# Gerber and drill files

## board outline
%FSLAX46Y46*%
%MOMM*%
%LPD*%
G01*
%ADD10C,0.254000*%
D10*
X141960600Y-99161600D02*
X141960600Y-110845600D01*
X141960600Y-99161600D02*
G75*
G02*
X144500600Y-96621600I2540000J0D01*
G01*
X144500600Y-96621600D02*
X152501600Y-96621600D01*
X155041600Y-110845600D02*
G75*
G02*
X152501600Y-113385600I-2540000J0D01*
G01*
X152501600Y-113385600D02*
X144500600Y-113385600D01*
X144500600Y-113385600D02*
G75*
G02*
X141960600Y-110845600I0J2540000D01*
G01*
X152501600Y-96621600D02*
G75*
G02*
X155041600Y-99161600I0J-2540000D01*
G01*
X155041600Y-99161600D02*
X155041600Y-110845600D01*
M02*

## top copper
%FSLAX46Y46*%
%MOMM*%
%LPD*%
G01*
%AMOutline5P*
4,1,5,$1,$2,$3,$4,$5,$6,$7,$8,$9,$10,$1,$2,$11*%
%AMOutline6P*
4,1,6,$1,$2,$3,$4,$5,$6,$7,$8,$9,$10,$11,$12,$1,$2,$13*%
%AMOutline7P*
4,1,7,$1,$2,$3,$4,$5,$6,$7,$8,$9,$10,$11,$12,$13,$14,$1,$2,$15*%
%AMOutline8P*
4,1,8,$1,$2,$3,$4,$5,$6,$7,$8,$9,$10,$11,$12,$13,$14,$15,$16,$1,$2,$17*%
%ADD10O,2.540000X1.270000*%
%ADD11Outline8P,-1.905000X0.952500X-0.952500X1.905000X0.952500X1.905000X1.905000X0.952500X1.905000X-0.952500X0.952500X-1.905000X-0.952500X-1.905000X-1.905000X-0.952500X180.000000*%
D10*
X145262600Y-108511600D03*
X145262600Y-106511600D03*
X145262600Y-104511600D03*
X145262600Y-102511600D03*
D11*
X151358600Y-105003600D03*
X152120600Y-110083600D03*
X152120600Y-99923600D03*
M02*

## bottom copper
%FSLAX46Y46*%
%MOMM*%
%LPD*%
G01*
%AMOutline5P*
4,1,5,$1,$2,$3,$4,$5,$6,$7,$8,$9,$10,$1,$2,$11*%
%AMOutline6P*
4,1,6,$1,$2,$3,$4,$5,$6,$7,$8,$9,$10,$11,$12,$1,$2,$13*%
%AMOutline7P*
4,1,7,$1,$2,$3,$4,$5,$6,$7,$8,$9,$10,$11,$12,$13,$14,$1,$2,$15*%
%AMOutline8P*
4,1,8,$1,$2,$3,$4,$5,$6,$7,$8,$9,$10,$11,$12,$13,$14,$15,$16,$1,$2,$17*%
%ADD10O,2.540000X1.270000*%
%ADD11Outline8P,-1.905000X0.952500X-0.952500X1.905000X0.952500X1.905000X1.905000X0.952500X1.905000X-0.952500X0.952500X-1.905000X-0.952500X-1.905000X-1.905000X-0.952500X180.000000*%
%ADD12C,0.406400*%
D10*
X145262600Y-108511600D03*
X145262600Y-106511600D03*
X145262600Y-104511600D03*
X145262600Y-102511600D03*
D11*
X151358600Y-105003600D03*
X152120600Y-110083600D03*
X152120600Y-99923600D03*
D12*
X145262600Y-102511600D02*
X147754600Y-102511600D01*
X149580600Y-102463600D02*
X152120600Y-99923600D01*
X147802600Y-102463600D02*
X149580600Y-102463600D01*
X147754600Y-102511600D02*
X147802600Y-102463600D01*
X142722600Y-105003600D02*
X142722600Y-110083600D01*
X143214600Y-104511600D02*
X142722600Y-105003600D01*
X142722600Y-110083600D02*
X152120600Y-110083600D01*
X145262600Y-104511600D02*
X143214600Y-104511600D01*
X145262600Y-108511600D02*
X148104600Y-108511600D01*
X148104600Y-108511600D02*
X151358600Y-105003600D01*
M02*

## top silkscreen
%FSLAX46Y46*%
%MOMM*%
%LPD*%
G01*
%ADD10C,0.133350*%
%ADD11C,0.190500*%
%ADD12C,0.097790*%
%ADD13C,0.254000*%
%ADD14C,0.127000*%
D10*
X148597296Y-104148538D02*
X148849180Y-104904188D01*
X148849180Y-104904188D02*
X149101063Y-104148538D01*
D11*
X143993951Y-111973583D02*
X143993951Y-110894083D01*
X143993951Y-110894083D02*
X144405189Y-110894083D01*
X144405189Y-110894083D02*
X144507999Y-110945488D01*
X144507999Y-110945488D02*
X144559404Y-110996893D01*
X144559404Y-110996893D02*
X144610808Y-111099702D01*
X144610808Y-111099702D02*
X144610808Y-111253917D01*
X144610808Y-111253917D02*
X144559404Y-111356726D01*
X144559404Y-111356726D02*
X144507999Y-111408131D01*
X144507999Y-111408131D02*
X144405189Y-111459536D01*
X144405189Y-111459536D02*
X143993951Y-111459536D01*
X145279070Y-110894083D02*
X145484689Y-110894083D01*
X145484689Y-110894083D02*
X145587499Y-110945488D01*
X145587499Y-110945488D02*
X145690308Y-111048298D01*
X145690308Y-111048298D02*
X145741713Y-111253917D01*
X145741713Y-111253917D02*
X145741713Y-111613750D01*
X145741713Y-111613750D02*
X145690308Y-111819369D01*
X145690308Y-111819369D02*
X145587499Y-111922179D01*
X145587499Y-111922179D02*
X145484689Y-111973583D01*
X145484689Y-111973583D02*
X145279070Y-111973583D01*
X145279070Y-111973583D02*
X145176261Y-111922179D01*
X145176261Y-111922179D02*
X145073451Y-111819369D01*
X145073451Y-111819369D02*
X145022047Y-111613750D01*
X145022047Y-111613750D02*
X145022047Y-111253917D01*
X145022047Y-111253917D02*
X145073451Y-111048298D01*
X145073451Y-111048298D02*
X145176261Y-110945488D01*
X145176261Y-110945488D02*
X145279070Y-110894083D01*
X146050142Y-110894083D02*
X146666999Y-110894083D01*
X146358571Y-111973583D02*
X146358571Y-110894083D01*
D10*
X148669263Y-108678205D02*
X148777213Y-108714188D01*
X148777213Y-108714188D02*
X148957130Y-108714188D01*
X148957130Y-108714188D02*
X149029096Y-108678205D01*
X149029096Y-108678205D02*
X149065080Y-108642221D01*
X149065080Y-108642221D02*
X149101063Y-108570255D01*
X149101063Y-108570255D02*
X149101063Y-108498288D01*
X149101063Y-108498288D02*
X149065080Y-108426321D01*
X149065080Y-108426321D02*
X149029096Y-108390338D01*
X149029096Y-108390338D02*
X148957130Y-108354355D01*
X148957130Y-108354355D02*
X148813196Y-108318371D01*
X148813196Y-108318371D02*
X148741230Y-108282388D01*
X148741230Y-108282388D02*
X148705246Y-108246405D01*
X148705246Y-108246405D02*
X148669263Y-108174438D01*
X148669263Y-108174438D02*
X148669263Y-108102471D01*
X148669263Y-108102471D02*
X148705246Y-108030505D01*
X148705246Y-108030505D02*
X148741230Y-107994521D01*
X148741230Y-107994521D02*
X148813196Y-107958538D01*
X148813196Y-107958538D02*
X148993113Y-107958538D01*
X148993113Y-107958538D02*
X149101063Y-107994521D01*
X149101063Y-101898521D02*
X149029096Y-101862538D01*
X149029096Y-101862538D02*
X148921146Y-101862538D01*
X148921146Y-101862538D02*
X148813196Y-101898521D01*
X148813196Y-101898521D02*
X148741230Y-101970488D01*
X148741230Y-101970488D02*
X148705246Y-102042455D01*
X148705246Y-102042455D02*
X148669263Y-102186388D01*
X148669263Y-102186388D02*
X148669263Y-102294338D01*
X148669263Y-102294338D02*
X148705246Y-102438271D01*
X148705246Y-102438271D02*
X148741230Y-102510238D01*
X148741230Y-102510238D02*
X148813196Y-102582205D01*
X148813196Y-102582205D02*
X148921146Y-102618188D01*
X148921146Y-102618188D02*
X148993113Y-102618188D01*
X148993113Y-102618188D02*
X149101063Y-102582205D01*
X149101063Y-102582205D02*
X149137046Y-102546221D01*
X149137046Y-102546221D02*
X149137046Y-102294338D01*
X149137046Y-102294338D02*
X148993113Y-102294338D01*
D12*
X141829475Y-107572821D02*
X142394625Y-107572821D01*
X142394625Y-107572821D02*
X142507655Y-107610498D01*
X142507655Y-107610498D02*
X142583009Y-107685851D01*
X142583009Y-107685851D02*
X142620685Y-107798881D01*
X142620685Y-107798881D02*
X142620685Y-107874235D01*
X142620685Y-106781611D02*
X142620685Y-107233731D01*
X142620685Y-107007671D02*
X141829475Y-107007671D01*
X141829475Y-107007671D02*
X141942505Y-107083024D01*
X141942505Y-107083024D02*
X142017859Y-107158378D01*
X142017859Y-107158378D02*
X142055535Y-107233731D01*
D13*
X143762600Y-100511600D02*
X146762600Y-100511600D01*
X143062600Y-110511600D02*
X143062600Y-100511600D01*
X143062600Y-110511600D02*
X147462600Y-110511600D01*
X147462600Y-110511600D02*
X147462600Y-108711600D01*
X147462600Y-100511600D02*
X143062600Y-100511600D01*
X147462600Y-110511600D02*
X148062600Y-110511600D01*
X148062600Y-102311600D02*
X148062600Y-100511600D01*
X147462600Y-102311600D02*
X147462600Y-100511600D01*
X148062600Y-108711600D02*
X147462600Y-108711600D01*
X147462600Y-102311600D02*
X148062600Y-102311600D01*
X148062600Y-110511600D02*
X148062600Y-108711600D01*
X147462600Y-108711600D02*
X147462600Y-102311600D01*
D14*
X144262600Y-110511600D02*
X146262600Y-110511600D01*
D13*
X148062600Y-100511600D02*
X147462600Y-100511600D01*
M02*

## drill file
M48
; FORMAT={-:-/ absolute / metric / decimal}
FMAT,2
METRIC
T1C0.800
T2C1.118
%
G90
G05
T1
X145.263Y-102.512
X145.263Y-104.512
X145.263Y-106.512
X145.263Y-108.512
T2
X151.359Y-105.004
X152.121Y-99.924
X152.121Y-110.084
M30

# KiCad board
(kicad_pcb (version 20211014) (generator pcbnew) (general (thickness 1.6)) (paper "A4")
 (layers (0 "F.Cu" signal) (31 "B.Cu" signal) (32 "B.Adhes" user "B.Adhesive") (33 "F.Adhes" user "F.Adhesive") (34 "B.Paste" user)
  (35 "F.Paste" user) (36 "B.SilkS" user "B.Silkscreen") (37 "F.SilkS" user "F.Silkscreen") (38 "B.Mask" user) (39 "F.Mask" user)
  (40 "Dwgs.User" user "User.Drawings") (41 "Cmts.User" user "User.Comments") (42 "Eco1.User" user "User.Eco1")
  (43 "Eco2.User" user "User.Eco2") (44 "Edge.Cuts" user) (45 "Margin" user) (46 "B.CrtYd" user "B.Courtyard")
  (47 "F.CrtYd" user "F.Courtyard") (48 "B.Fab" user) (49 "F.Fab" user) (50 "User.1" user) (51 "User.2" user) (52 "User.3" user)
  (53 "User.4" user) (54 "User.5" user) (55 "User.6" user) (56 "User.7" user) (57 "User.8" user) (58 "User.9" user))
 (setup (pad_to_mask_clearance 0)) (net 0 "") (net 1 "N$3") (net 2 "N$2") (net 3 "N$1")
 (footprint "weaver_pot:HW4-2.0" (layer "F.Cu") (at 145.2626 105.5116 90)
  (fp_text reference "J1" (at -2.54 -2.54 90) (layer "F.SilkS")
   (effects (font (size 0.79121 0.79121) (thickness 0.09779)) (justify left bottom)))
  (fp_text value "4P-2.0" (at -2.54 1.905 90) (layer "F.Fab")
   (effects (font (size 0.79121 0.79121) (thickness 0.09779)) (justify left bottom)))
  (fp_line (start 5 -1.5) (end 5 1.5) (layer "F.SilkS") (width 0.254))
  (fp_line (start -5 -2.2) (end 5 -2.2) (layer "F.SilkS") (width 0.254))
  (fp_line (start -5 -2.2) (end -5 2.2) (layer "F.SilkS") (width 0.254))
  (fp_line (start -5 2.2) (end -3.2 2.2) (layer "F.SilkS") (width 0.254))
  (fp_line (start 5 2.2) (end 5 -2.2) (layer "F.SilkS") (width 0.254))
  (fp_line (start -5 2.2) (end -5 2.8) (layer "F.SilkS") (width 0.254))
  (fp_line (start 3.2 2.8) (end 5 2.8) (layer "F.SilkS") (width 0.254))
  (fp_line (start 3.2 2.2) (end 5 2.2) (layer "F.SilkS") (width 0.254))
  (fp_line (start -3.2 2.8) (end -3.2 2.2) (layer "F.SilkS") (width 0.254))
  (fp_line (start 3.2 2.2) (end 3.2 2.8) (layer "F.SilkS") (width 0.254))
  (fp_line (start -5 2.8) (end -3.2 2.8) (layer "F.SilkS") (width 0.254))
  (fp_line (start -3.2 2.2) (end 3.2 2.2) (layer "F.SilkS") (width 0.254))
  (fp_line (start -5 -1) (end -5 1) (layer "F.SilkS") (width 0.127))
  (fp_line (start 5 2.8) (end 5 2.2) (layer "F.SilkS") (width 0.254))
  (pad "1" thru_hole oval (at -3 0 180) (size 2.54 1.27) (drill 0.8) (layers *.Cu *.Mask) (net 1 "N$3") (solder_mask_margin 0.1016))
  (pad "2" thru_hole oval (at -1 0 180) (size 2.54 1.27) (drill 0.8) (layers *.Cu *.Mask) (solder_mask_margin 0.1016))
  (pad "3" thru_hole oval (at 1 0 180) (size 2.54 1.27) (drill 0.8) (layers *.Cu *.Mask) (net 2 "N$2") (solder_mask_margin 0.1016))
  (pad "4" thru_hole oval (at 3 0 180) (size 2.54 1.27) (drill 0.8) (layers *.Cu *.Mask) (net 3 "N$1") (solder_mask_margin 0.1016)))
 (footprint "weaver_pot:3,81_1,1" (layer "B.Cu") (at 151.3586 105.0036 180)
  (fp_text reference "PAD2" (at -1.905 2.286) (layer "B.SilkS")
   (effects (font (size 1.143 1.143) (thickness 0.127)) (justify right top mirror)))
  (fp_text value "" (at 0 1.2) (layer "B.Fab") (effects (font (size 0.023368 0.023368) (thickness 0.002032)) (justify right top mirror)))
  (pad "1" thru_hole roundrect (at 0 0 180) (size 3.81 3.81) (drill 1.1176) (layers *.Cu *.Mask) (roundrect_rratio 0.25)
   (chamfer_ratio 0.25) (chamfer top_left top_right bottom_left bottom_right) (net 1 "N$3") (solder_mask_margin 0.1016)))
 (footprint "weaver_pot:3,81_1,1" (layer "B.Cu") (at 152.1206 110.0836 180)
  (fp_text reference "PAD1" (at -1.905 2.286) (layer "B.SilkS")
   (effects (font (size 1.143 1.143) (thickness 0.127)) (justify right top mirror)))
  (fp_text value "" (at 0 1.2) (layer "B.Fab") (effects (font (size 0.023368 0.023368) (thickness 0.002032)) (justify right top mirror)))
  (pad "1" thru_hole roundrect (at 0 0 180) (size 3.81 3.81) (drill 1.1176) (layers *.Cu *.Mask) (roundrect_rratio 0.25)
   (chamfer_ratio 0.25) (chamfer top_left top_right bottom_left bottom_right) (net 2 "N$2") (solder_mask_margin 0.1016)))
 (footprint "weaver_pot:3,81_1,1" (layer "B.Cu") (at 152.1206 99.9236 180)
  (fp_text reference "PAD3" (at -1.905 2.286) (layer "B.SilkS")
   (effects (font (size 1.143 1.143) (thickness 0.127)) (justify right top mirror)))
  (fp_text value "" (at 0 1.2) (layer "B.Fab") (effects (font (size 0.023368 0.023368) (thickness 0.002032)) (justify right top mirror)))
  (pad "1" thru_hole roundrect (at 0 0 180) (size 3.81 3.81) (drill 1.1176) (layers *.Cu *.Mask) (roundrect_rratio 0.25)
   (chamfer_ratio 0.25) (chamfer top_left top_right bottom_left bottom_right) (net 3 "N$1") (solder_mask_margin 0.1016)))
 (gr_line (start 141.9606 99.1616) (end 141.9606 110.8456) (layer "Edge.Cuts") (width 0.254))
 (gr_arc (start 141.9606 99.1616) (mid 142.704549 97.365549) (end 144.5006 96.6216) (layer "Edge.Cuts") (width 0.254))
 (gr_line (start 144.5006 96.6216) (end 152.5016 96.6216) (layer "Edge.Cuts") (width 0.254))
 (gr_arc (start 155.0416 110.8456) (mid 154.297651 112.641651) (end 152.5016 113.3856) (layer "Edge.Cuts") (width 0.254))
 (gr_line (start 152.5016 113.3856) (end 144.5006 113.3856) (layer "Edge.Cuts") (width 0.254))
 (gr_arc (start 144.5006 113.3856) (mid 142.704549 112.641651) (end 141.9606 110.8456) (layer "Edge.Cuts") (width 0.254))
 (gr_arc (start 152.5016 96.6216) (mid 154.297651 97.365549) (end 155.0416 99.1616) (layer "Edge.Cuts") (width 0.254))
 (gr_line (start 155.0416 99.1616) (end 155.0416 110.8456) (layer "Edge.Cuts") (width 0.254))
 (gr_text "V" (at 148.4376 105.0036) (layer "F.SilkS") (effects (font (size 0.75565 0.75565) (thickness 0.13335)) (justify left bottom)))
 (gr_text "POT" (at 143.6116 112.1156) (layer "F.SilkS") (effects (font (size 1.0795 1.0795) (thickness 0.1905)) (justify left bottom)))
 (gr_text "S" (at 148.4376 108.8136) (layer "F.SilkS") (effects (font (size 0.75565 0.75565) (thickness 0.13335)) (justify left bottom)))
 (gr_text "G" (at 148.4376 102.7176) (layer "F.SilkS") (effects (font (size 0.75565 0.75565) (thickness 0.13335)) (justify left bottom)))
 (segment (start 145.2626 102.5116) (end 147.7546 102.5116) (width 0.4064) (layer "B.Cu") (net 3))
 (segment (start 149.5806 102.4636) (end 152.1206 99.9236) (width 0.4064) (layer "B.Cu") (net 3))
 (segment (start 147.8026 102.4636) (end 149.5806 102.4636) (width 0.4064) (layer "B.Cu") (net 3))
 (segment (start 147.7546 102.5116) (end 147.8026 102.4636) (width 0.4064) (layer "B.Cu") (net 3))
 (segment (start 142.7226 105.0036) (end 142.7226 110.0836) (width 0.4064) (layer "B.Cu") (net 2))
 (segment (start 143.2146 104.5116) (end 142.7226 105.0036) (width 0.4064) (layer "B.Cu") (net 2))
 (segment (start 142.7226 110.0836) (end 152.1206 110.0836) (width 0.4064) (layer "B.Cu") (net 2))
 (segment (start 145.2626 104.5116) (end 143.2146 104.5116) (width 0.4064) (layer "B.Cu") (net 2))
 (segment (start 145.2626 108.5116) (end 148.1046 108.5116) (width 0.4064) (layer "B.Cu") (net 1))
 (segment (start 148.1046 108.5116) (end 151.3586 105.0036) (width 0.4064) (layer "B.Cu") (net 1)))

